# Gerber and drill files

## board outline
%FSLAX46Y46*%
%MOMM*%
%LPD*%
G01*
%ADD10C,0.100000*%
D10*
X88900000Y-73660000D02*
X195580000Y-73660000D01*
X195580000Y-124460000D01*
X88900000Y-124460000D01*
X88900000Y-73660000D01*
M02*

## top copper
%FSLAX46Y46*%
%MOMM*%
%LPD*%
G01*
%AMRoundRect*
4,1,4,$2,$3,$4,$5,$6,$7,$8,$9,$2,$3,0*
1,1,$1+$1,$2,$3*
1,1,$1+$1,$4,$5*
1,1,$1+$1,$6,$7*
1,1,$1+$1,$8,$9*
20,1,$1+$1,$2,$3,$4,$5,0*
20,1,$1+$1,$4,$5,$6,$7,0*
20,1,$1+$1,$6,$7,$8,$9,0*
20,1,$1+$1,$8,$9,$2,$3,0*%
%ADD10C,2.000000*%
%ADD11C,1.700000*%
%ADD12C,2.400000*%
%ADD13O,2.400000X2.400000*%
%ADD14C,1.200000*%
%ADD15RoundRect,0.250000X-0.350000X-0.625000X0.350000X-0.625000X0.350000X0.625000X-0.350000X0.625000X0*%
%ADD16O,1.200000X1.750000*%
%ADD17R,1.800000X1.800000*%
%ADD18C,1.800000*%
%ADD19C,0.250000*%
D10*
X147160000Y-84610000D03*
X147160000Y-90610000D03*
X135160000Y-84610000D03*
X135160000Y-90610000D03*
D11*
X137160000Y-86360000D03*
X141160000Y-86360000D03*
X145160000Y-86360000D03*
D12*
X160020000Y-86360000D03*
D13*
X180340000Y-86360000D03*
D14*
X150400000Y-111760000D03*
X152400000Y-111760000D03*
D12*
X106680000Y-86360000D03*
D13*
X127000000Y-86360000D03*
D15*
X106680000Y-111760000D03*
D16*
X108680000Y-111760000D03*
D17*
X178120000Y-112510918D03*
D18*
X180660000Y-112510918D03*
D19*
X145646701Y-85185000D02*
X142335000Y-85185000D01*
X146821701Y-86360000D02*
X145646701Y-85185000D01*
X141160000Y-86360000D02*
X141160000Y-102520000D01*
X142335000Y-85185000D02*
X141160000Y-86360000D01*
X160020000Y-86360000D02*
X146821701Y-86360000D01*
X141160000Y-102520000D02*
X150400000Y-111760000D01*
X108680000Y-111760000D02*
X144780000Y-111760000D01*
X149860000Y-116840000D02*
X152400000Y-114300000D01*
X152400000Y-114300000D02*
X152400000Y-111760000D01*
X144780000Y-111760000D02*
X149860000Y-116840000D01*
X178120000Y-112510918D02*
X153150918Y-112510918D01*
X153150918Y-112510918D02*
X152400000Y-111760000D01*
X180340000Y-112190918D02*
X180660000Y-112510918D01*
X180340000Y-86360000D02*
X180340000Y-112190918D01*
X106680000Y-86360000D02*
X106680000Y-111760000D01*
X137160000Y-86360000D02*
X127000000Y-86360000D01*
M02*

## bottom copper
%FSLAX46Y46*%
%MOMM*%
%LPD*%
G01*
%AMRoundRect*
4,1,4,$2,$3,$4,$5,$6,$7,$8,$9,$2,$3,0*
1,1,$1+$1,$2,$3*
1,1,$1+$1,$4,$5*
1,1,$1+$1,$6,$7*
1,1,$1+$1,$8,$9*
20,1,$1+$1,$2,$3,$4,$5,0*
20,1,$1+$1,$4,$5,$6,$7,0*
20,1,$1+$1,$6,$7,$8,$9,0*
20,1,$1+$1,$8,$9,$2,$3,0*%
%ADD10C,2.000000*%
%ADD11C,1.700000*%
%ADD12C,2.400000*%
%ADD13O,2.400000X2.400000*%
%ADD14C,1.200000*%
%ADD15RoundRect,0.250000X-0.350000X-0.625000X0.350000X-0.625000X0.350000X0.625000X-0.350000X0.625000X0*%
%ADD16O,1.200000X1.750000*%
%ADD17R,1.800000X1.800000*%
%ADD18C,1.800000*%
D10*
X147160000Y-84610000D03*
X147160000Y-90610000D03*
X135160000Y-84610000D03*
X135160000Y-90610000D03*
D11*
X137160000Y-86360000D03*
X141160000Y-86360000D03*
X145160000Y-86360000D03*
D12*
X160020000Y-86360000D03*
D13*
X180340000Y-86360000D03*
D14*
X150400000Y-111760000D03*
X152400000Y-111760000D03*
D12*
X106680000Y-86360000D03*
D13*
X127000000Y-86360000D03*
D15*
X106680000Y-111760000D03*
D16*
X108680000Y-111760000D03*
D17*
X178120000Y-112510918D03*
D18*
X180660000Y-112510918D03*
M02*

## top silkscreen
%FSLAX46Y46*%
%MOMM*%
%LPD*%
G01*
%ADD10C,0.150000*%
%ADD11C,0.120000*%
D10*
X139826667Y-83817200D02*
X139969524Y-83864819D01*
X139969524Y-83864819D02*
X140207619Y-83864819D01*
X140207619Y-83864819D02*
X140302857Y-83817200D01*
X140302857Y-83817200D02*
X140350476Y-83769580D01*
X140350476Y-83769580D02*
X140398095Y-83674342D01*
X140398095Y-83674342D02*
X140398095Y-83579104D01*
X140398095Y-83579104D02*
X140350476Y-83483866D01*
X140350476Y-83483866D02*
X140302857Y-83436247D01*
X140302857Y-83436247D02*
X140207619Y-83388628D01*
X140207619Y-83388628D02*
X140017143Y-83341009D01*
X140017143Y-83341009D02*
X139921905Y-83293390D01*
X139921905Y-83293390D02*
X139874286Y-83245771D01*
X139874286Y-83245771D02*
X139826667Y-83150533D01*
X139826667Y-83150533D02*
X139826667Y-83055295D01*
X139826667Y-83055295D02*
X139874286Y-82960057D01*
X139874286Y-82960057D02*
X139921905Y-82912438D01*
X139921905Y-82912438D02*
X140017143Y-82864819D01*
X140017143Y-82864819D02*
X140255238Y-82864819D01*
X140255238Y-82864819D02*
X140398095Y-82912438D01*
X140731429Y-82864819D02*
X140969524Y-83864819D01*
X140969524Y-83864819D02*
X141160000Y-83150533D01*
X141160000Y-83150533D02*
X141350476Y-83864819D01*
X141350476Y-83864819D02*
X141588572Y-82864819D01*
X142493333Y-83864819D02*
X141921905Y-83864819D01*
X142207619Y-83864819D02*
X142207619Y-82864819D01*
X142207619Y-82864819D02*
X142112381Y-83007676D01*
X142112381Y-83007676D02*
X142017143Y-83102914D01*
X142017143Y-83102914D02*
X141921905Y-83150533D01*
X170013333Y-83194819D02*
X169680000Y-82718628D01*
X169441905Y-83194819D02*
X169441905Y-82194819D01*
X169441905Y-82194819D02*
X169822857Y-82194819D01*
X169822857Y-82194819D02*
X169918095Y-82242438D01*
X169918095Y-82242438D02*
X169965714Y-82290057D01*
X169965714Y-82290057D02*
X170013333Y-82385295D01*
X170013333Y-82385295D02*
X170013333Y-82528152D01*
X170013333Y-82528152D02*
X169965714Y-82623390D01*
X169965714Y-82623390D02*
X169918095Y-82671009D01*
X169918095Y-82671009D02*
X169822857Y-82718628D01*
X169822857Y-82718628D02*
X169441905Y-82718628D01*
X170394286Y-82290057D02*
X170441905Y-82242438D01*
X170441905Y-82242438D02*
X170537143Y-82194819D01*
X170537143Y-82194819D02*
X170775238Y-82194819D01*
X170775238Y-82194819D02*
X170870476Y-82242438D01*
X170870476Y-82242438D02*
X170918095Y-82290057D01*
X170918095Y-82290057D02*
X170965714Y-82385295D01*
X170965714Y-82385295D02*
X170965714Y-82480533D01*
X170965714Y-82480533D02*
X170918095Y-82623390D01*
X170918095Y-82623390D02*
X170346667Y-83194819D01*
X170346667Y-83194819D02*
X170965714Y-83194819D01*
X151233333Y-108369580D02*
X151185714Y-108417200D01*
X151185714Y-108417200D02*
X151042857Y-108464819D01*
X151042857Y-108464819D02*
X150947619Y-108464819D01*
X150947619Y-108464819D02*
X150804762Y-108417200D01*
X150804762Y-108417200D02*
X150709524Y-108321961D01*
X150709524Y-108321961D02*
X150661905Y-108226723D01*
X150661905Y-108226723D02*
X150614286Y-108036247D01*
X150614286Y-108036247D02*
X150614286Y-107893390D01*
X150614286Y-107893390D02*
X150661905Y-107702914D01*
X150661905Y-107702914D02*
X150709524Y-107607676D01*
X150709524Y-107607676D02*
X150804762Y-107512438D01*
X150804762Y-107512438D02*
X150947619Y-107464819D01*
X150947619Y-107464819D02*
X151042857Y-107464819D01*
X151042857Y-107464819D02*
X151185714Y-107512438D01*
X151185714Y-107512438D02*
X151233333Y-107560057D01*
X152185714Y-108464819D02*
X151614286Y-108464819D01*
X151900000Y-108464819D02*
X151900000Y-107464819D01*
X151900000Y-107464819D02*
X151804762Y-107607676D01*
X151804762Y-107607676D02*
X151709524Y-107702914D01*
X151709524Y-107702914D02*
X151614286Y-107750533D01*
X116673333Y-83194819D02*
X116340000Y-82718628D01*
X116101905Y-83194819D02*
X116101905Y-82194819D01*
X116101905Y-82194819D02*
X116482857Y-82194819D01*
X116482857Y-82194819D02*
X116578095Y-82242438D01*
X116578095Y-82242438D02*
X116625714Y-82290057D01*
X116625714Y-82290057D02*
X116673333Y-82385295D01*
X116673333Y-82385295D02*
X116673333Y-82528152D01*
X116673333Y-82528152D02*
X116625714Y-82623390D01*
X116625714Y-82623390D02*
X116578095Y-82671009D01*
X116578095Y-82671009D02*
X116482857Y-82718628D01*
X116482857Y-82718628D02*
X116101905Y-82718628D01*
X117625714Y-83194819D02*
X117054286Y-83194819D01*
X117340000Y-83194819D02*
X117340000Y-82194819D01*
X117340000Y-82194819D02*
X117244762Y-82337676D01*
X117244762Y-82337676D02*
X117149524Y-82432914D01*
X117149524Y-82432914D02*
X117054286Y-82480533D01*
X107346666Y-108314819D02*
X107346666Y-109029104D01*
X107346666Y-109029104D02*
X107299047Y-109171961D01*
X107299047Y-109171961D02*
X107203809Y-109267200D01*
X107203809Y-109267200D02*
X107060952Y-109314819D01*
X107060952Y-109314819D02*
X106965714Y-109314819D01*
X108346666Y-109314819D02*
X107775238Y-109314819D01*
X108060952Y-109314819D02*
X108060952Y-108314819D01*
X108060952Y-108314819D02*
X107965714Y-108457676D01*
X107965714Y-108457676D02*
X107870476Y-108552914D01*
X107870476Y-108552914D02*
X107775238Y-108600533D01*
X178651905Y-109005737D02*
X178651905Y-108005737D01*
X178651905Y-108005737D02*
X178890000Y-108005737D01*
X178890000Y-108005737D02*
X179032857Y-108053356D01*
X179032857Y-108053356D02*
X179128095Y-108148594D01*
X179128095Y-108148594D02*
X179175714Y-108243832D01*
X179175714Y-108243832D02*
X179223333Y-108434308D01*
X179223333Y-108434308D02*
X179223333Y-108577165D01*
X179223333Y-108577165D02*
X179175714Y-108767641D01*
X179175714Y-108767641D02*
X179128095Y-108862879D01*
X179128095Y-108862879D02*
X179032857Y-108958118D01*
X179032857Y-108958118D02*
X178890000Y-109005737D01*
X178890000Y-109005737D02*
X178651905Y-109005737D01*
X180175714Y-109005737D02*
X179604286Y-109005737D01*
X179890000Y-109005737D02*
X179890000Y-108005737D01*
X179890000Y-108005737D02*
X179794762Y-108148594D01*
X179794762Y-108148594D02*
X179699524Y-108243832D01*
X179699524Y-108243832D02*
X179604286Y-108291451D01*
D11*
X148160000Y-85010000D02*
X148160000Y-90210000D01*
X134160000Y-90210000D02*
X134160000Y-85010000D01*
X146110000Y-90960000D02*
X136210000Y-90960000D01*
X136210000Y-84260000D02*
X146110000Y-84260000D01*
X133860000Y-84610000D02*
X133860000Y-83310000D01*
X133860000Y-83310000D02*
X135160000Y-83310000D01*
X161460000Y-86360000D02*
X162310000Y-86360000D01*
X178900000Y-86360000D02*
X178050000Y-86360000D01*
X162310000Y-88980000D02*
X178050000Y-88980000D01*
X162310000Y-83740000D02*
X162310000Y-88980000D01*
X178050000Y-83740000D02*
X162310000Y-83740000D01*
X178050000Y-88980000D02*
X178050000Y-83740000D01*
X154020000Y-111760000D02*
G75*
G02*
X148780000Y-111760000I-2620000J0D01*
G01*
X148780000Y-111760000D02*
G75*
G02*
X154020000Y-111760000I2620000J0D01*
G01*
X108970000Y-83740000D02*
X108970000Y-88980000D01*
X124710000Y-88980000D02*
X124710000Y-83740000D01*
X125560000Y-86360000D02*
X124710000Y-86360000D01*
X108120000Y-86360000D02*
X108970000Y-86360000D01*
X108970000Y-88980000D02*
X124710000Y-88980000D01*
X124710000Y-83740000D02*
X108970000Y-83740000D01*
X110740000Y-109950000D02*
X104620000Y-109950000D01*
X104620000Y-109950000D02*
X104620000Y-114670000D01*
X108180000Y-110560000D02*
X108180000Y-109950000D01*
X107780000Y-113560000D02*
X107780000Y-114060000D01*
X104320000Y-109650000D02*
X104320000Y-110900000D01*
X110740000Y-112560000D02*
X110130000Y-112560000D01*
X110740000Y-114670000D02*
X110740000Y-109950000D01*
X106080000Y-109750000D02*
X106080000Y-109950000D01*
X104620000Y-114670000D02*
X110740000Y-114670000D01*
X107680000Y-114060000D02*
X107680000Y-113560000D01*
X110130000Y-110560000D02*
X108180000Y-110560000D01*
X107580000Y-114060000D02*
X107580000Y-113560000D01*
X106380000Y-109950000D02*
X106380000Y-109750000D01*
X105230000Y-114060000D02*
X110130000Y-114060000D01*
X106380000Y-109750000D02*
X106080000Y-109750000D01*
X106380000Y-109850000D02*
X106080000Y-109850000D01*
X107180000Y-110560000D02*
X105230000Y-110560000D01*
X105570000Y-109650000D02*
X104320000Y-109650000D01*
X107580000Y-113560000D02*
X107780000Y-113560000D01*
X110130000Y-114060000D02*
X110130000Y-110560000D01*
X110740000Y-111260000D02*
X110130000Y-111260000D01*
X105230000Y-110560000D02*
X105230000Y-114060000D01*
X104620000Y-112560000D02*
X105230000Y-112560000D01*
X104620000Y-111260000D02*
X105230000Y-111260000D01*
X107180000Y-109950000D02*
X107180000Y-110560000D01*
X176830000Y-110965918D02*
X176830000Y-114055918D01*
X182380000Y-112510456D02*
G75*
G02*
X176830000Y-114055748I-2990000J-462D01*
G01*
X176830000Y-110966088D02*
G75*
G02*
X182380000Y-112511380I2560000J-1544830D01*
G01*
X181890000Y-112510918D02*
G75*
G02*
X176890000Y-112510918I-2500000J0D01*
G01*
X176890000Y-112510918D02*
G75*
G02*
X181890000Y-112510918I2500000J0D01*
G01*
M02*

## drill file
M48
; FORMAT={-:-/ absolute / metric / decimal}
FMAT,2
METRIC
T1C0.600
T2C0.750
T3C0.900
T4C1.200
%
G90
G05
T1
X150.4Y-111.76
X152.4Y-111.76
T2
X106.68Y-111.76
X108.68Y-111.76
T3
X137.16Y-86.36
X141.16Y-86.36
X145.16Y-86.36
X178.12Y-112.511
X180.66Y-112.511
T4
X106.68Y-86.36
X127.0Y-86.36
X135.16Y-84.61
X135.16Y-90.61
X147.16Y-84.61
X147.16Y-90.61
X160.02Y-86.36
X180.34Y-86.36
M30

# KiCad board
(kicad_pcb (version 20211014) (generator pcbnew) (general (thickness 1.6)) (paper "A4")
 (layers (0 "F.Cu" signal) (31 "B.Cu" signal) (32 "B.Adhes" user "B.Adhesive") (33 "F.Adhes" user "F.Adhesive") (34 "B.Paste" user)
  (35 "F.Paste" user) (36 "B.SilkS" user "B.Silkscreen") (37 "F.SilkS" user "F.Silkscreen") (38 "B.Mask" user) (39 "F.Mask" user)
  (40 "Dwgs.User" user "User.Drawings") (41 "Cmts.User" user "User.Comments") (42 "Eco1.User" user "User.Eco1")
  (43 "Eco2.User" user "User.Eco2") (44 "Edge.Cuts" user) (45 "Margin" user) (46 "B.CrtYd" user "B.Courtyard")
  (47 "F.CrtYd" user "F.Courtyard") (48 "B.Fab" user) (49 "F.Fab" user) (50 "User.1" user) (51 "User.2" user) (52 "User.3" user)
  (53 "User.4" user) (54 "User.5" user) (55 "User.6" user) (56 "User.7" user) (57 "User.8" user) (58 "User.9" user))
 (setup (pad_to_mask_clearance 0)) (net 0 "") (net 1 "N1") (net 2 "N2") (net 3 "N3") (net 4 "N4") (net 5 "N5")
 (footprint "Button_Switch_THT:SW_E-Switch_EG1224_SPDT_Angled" (layer "F.Cu") (at 137.16 86.36)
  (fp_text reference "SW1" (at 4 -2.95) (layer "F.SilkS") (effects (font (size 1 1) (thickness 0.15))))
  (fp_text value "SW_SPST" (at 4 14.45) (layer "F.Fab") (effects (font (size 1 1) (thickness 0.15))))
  (fp_line (start 11 -1.35) (end 11 3.85) (layer "F.SilkS") (width 0.12))
  (fp_line (start -3 3.85) (end -3 -1.35) (layer "F.SilkS") (width 0.12))
  (fp_line (start 8.95 4.6) (end -0.95 4.6) (layer "F.SilkS") (width 0.12))
  (fp_line (start -0.95 -2.1) (end 8.95 -2.1) (layer "F.SilkS") (width 0.12))
  (fp_line (start -3.3 -1.75) (end -3.3 -3.05) (layer "F.SilkS") (width 0.12))
  (fp_line (start -3.3 -3.05) (end -2 -3.05) (layer "F.SilkS") (width 0.12))
  (pad "" thru_hole circle (at 10 -1.75) (size 2 2) (drill 1.2) (layers *.Cu *.Mask))
  (pad "" thru_hole circle (at 10 4.25) (size 2 2) (drill 1.2) (layers *.Cu *.Mask))
  (pad "" thru_hole circle (at -2 -1.75) (size 2 2) (drill 1.2) (layers *.Cu *.Mask))
  (pad "" thru_hole circle (at -2 4.25) (size 2 2) (drill 1.2) (layers *.Cu *.Mask))
  (pad "1" thru_hole circle (at 0 0) (size 1.7 1.7) (drill 0.9) (layers *.Cu *.Mask) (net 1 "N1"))
  (pad "2" thru_hole circle (at 4 0) (size 1.7 1.7) (drill 0.9) (layers *.Cu *.Mask) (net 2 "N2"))
  (pad "3" thru_hole circle (at 8 0) (size 1.7 1.7) (drill 0.9) (layers *.Cu *.Mask)))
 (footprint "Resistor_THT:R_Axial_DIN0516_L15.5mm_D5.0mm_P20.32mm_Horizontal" (layer "F.Cu") (at 160.02 86.36)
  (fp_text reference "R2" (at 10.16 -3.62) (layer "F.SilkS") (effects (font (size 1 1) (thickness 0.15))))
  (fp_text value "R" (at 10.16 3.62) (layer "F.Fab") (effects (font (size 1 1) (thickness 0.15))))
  (fp_line (start 1.44 0) (end 2.29 0) (layer "F.SilkS") (width 0.12))
  (fp_line (start 18.88 0) (end 18.03 0) (layer "F.SilkS") (width 0.12))
  (fp_line (start 2.29 2.62) (end 18.03 2.62) (layer "F.SilkS") (width 0.12))
  (fp_line (start 2.29 -2.62) (end 2.29 2.62) (layer "F.SilkS") (width 0.12))
  (fp_line (start 18.03 -2.62) (end 2.29 -2.62) (layer "F.SilkS") (width 0.12))
  (fp_line (start 18.03 2.62) (end 18.03 -2.62) (layer "F.SilkS") (width 0.12))
  (pad "1" thru_hole circle (at 0 0) (size 2.4 2.4) (drill 1.2) (layers *.Cu *.Mask) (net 2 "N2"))
  (pad "2" thru_hole oval (at 20.32 0) (size 2.4 2.4) (drill 1.2) (layers *.Cu *.Mask) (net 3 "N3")))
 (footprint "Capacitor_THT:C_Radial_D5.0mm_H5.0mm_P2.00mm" (layer "F.Cu") (at 150.4 111.76)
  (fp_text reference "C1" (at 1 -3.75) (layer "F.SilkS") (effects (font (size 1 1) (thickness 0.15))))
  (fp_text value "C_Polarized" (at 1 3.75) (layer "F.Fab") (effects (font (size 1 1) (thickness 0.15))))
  (fp_circle (center 1 0) (end 3.62 0) (layer "F.SilkS") (width 0.12) (fill none))
  (pad "1" thru_hole circle (at 0 0) (size 1.2 1.2) (drill 0.6) (layers *.Cu *.Mask) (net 2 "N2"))
  (pad "2" thru_hole circle (at 2 0) (size 1.2 1.2) (drill 0.6) (layers *.Cu *.Mask) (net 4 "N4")))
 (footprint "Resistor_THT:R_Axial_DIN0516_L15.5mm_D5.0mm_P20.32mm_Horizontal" (layer "F.Cu") (at 106.68 86.36)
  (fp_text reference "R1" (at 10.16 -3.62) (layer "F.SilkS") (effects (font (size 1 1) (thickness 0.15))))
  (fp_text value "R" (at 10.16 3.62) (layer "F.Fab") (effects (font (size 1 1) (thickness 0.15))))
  (fp_line (start 2.29 -2.62) (end 2.29 2.62) (layer "F.SilkS") (width 0.12))
  (fp_line (start 18.03 2.62) (end 18.03 -2.62) (layer "F.SilkS") (width 0.12))
  (fp_line (start 18.88 0) (end 18.03 0) (layer "F.SilkS") (width 0.12))
  (fp_line (start 1.44 0) (end 2.29 0) (layer "F.SilkS") (width 0.12))
  (fp_line (start 2.29 2.62) (end 18.03 2.62) (layer "F.SilkS") (width 0.12))
  (fp_line (start 18.03 -2.62) (end 2.29 -2.62) (layer "F.SilkS") (width 0.12))
  (pad "1" thru_hole circle (at 0 0) (size 2.4 2.4) (drill 1.2) (layers *.Cu *.Mask) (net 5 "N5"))
  (pad "2" thru_hole oval (at 20.32 0) (size 2.4 2.4) (drill 1.2) (layers *.Cu *.Mask) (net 1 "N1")))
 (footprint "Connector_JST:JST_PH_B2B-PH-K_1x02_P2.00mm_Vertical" (layer "F.Cu") (at 106.68 111.76)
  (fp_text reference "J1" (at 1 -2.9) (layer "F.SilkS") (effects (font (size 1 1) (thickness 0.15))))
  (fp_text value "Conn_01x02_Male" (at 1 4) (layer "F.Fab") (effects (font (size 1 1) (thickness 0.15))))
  (fp_line (start 4.06 -1.81) (end -2.06 -1.81) (layer "F.SilkS") (width 0.12))
  (fp_line (start -2.06 -1.81) (end -2.06 2.91) (layer "F.SilkS") (width 0.12))
  (fp_line (start 1.5 -1.2) (end 1.5 -1.81) (layer "F.SilkS") (width 0.12))
  (fp_line (start 1.1 1.8) (end 1.1 2.3) (layer "F.SilkS") (width 0.12))
  (fp_line (start -2.36 -2.11) (end -2.36 -0.86) (layer "F.SilkS") (width 0.12))
  (fp_line (start 4.06 0.8) (end 3.45 0.8) (layer "F.SilkS") (width 0.12))
  (fp_line (start 4.06 2.91) (end 4.06 -1.81) (layer "F.SilkS") (width 0.12))
  (fp_line (start -0.6 -2.01) (end -0.6 -1.81) (layer "F.SilkS") (width 0.12))
  (fp_line (start -2.06 2.91) (end 4.06 2.91) (layer "F.SilkS") (width 0.12))
  (fp_line (start 1 2.3) (end 1 1.8) (layer "F.SilkS") (width 0.12))
  (fp_line (start 3.45 -1.2) (end 1.5 -1.2) (layer "F.SilkS") (width 0.12))
  (fp_line (start 0.9 2.3) (end 0.9 1.8) (layer "F.SilkS") (width 0.12))
  (fp_line (start -0.3 -1.81) (end -0.3 -2.01) (layer "F.SilkS") (width 0.12))
  (fp_line (start -1.45 2.3) (end 3.45 2.3) (layer "F.SilkS") (width 0.12))
  (fp_line (start -0.3 -2.01) (end -0.6 -2.01) (layer "F.SilkS") (width 0.12))
  (fp_line (start -0.3 -1.91) (end -0.6 -1.91) (layer "F.SilkS") (width 0.12))
  (fp_line (start 0.5 -1.2) (end -1.45 -1.2) (layer "F.SilkS") (width 0.12))
  (fp_line (start -1.11 -2.11) (end -2.36 -2.11) (layer "F.SilkS") (width 0.12))
  (fp_line (start 0.9 1.8) (end 1.1 1.8) (layer "F.SilkS") (width 0.12))
  (fp_line (start 3.45 2.3) (end 3.45 -1.2) (layer "F.SilkS") (width 0.12))
  (fp_line (start 4.06 -0.5) (end 3.45 -0.5) (layer "F.SilkS") (width 0.12))
  (fp_line (start -1.45 -1.2) (end -1.45 2.3) (layer "F.SilkS") (width 0.12))
  (fp_line (start -2.06 0.8) (end -1.45 0.8) (layer "F.SilkS") (width 0.12))
  (fp_line (start -2.06 -0.5) (end -1.45 -0.5) (layer "F.SilkS") (width 0.12))
  (fp_line (start 0.5 -1.81) (end 0.5 -1.2) (layer "F.SilkS") (width 0.12))
  (pad "1" thru_hole roundrect (at 0 0) (size 1.2 1.75) (drill 0.75) (layers *.Cu *.Mask) (roundrect_rratio 0.208333) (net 5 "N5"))
  (pad "2" thru_hole oval (at 2 0) (size 1.2 1.75) (drill 0.75) (layers *.Cu *.Mask) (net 4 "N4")))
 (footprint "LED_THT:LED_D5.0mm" (layer "F.Cu") (at 178.12 112.510918)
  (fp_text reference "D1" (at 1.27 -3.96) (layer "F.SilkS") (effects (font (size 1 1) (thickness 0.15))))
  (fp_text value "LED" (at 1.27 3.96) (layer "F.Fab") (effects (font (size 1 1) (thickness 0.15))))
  (fp_line (start -1.29 -1.545) (end -1.29 1.545) (layer "F.SilkS") (width 0.12))
  (fp_arc (start 4.26 -0.000462) (mid 2.072002 2.880433) (end -1.29 1.54483) (layer "F.SilkS") (width 0.12))
  (fp_arc (start -1.29 -1.54483) (mid 2.072002 -2.880433) (end 4.26 0.000462) (layer "F.SilkS") (width 0.12))
  (fp_circle (center 1.27 0) (end 3.77 0) (layer "F.SilkS") (width 0.12) (fill none))
  (pad "1" thru_hole rect (at 0 0) (size 1.8 1.8) (drill 0.9) (layers *.Cu *.Mask) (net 4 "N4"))
  (pad "2" thru_hole circle (at 2.54 0) (size 1.8 1.8) (drill 0.9) (layers *.Cu *.Mask) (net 3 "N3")))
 (gr_rect (start 88.9 73.66) (end 195.58 124.46) (layer "Edge.Cuts") (width 0.1) (fill none))
 (segment (start 145.646701 85.185) (end 142.335 85.185) (width 0.25) (layer "F.Cu") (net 2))
 (segment (start 146.821701 86.36) (end 145.646701 85.185) (width 0.25) (layer "F.Cu") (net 2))
 (segment (start 141.16 86.36) (end 141.16 102.52) (width 0.25) (layer "F.Cu") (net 2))
 (segment (start 142.335 85.185) (end 141.16 86.36) (width 0.25) (layer "F.Cu") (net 2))
 (segment (start 160.02 86.36) (end 146.821701 86.36) (width 0.25) (layer "F.Cu") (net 2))
 (segment (start 141.16 102.52) (end 150.4 111.76) (width 0.25) (layer "F.Cu") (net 2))
 (segment (start 108.68 111.76) (end 144.78 111.76) (width 0.25) (layer "F.Cu") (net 4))
 (segment (start 149.86 116.84) (end 152.4 114.3) (width 0.25) (layer "F.Cu") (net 4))
 (segment (start 152.4 114.3) (end 152.4 111.76) (width 0.25) (layer "F.Cu") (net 4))
 (segment (start 144.78 111.76) (end 149.86 116.84) (width 0.25) (layer "F.Cu") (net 4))
 (segment (start 178.12 112.510918) (end 153.150918 112.510918) (width 0.25) (layer "F.Cu") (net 4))
 (segment (start 153.150918 112.510918) (end 152.4 111.76) (width 0.25) (layer "F.Cu") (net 4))
 (segment (start 180.34 112.190918) (end 180.66 112.510918) (width 0.25) (layer "F.Cu") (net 3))
 (segment (start 180.34 86.36) (end 180.34 112.190918) (width 0.25) (layer "F.Cu") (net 3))
 (segment (start 106.68 86.36) (end 106.68 111.76) (width 0.25) (layer "F.Cu") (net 5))
 (segment (start 137.16 86.36) (end 127 86.36) (width 0.25) (layer "F.Cu") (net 1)))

